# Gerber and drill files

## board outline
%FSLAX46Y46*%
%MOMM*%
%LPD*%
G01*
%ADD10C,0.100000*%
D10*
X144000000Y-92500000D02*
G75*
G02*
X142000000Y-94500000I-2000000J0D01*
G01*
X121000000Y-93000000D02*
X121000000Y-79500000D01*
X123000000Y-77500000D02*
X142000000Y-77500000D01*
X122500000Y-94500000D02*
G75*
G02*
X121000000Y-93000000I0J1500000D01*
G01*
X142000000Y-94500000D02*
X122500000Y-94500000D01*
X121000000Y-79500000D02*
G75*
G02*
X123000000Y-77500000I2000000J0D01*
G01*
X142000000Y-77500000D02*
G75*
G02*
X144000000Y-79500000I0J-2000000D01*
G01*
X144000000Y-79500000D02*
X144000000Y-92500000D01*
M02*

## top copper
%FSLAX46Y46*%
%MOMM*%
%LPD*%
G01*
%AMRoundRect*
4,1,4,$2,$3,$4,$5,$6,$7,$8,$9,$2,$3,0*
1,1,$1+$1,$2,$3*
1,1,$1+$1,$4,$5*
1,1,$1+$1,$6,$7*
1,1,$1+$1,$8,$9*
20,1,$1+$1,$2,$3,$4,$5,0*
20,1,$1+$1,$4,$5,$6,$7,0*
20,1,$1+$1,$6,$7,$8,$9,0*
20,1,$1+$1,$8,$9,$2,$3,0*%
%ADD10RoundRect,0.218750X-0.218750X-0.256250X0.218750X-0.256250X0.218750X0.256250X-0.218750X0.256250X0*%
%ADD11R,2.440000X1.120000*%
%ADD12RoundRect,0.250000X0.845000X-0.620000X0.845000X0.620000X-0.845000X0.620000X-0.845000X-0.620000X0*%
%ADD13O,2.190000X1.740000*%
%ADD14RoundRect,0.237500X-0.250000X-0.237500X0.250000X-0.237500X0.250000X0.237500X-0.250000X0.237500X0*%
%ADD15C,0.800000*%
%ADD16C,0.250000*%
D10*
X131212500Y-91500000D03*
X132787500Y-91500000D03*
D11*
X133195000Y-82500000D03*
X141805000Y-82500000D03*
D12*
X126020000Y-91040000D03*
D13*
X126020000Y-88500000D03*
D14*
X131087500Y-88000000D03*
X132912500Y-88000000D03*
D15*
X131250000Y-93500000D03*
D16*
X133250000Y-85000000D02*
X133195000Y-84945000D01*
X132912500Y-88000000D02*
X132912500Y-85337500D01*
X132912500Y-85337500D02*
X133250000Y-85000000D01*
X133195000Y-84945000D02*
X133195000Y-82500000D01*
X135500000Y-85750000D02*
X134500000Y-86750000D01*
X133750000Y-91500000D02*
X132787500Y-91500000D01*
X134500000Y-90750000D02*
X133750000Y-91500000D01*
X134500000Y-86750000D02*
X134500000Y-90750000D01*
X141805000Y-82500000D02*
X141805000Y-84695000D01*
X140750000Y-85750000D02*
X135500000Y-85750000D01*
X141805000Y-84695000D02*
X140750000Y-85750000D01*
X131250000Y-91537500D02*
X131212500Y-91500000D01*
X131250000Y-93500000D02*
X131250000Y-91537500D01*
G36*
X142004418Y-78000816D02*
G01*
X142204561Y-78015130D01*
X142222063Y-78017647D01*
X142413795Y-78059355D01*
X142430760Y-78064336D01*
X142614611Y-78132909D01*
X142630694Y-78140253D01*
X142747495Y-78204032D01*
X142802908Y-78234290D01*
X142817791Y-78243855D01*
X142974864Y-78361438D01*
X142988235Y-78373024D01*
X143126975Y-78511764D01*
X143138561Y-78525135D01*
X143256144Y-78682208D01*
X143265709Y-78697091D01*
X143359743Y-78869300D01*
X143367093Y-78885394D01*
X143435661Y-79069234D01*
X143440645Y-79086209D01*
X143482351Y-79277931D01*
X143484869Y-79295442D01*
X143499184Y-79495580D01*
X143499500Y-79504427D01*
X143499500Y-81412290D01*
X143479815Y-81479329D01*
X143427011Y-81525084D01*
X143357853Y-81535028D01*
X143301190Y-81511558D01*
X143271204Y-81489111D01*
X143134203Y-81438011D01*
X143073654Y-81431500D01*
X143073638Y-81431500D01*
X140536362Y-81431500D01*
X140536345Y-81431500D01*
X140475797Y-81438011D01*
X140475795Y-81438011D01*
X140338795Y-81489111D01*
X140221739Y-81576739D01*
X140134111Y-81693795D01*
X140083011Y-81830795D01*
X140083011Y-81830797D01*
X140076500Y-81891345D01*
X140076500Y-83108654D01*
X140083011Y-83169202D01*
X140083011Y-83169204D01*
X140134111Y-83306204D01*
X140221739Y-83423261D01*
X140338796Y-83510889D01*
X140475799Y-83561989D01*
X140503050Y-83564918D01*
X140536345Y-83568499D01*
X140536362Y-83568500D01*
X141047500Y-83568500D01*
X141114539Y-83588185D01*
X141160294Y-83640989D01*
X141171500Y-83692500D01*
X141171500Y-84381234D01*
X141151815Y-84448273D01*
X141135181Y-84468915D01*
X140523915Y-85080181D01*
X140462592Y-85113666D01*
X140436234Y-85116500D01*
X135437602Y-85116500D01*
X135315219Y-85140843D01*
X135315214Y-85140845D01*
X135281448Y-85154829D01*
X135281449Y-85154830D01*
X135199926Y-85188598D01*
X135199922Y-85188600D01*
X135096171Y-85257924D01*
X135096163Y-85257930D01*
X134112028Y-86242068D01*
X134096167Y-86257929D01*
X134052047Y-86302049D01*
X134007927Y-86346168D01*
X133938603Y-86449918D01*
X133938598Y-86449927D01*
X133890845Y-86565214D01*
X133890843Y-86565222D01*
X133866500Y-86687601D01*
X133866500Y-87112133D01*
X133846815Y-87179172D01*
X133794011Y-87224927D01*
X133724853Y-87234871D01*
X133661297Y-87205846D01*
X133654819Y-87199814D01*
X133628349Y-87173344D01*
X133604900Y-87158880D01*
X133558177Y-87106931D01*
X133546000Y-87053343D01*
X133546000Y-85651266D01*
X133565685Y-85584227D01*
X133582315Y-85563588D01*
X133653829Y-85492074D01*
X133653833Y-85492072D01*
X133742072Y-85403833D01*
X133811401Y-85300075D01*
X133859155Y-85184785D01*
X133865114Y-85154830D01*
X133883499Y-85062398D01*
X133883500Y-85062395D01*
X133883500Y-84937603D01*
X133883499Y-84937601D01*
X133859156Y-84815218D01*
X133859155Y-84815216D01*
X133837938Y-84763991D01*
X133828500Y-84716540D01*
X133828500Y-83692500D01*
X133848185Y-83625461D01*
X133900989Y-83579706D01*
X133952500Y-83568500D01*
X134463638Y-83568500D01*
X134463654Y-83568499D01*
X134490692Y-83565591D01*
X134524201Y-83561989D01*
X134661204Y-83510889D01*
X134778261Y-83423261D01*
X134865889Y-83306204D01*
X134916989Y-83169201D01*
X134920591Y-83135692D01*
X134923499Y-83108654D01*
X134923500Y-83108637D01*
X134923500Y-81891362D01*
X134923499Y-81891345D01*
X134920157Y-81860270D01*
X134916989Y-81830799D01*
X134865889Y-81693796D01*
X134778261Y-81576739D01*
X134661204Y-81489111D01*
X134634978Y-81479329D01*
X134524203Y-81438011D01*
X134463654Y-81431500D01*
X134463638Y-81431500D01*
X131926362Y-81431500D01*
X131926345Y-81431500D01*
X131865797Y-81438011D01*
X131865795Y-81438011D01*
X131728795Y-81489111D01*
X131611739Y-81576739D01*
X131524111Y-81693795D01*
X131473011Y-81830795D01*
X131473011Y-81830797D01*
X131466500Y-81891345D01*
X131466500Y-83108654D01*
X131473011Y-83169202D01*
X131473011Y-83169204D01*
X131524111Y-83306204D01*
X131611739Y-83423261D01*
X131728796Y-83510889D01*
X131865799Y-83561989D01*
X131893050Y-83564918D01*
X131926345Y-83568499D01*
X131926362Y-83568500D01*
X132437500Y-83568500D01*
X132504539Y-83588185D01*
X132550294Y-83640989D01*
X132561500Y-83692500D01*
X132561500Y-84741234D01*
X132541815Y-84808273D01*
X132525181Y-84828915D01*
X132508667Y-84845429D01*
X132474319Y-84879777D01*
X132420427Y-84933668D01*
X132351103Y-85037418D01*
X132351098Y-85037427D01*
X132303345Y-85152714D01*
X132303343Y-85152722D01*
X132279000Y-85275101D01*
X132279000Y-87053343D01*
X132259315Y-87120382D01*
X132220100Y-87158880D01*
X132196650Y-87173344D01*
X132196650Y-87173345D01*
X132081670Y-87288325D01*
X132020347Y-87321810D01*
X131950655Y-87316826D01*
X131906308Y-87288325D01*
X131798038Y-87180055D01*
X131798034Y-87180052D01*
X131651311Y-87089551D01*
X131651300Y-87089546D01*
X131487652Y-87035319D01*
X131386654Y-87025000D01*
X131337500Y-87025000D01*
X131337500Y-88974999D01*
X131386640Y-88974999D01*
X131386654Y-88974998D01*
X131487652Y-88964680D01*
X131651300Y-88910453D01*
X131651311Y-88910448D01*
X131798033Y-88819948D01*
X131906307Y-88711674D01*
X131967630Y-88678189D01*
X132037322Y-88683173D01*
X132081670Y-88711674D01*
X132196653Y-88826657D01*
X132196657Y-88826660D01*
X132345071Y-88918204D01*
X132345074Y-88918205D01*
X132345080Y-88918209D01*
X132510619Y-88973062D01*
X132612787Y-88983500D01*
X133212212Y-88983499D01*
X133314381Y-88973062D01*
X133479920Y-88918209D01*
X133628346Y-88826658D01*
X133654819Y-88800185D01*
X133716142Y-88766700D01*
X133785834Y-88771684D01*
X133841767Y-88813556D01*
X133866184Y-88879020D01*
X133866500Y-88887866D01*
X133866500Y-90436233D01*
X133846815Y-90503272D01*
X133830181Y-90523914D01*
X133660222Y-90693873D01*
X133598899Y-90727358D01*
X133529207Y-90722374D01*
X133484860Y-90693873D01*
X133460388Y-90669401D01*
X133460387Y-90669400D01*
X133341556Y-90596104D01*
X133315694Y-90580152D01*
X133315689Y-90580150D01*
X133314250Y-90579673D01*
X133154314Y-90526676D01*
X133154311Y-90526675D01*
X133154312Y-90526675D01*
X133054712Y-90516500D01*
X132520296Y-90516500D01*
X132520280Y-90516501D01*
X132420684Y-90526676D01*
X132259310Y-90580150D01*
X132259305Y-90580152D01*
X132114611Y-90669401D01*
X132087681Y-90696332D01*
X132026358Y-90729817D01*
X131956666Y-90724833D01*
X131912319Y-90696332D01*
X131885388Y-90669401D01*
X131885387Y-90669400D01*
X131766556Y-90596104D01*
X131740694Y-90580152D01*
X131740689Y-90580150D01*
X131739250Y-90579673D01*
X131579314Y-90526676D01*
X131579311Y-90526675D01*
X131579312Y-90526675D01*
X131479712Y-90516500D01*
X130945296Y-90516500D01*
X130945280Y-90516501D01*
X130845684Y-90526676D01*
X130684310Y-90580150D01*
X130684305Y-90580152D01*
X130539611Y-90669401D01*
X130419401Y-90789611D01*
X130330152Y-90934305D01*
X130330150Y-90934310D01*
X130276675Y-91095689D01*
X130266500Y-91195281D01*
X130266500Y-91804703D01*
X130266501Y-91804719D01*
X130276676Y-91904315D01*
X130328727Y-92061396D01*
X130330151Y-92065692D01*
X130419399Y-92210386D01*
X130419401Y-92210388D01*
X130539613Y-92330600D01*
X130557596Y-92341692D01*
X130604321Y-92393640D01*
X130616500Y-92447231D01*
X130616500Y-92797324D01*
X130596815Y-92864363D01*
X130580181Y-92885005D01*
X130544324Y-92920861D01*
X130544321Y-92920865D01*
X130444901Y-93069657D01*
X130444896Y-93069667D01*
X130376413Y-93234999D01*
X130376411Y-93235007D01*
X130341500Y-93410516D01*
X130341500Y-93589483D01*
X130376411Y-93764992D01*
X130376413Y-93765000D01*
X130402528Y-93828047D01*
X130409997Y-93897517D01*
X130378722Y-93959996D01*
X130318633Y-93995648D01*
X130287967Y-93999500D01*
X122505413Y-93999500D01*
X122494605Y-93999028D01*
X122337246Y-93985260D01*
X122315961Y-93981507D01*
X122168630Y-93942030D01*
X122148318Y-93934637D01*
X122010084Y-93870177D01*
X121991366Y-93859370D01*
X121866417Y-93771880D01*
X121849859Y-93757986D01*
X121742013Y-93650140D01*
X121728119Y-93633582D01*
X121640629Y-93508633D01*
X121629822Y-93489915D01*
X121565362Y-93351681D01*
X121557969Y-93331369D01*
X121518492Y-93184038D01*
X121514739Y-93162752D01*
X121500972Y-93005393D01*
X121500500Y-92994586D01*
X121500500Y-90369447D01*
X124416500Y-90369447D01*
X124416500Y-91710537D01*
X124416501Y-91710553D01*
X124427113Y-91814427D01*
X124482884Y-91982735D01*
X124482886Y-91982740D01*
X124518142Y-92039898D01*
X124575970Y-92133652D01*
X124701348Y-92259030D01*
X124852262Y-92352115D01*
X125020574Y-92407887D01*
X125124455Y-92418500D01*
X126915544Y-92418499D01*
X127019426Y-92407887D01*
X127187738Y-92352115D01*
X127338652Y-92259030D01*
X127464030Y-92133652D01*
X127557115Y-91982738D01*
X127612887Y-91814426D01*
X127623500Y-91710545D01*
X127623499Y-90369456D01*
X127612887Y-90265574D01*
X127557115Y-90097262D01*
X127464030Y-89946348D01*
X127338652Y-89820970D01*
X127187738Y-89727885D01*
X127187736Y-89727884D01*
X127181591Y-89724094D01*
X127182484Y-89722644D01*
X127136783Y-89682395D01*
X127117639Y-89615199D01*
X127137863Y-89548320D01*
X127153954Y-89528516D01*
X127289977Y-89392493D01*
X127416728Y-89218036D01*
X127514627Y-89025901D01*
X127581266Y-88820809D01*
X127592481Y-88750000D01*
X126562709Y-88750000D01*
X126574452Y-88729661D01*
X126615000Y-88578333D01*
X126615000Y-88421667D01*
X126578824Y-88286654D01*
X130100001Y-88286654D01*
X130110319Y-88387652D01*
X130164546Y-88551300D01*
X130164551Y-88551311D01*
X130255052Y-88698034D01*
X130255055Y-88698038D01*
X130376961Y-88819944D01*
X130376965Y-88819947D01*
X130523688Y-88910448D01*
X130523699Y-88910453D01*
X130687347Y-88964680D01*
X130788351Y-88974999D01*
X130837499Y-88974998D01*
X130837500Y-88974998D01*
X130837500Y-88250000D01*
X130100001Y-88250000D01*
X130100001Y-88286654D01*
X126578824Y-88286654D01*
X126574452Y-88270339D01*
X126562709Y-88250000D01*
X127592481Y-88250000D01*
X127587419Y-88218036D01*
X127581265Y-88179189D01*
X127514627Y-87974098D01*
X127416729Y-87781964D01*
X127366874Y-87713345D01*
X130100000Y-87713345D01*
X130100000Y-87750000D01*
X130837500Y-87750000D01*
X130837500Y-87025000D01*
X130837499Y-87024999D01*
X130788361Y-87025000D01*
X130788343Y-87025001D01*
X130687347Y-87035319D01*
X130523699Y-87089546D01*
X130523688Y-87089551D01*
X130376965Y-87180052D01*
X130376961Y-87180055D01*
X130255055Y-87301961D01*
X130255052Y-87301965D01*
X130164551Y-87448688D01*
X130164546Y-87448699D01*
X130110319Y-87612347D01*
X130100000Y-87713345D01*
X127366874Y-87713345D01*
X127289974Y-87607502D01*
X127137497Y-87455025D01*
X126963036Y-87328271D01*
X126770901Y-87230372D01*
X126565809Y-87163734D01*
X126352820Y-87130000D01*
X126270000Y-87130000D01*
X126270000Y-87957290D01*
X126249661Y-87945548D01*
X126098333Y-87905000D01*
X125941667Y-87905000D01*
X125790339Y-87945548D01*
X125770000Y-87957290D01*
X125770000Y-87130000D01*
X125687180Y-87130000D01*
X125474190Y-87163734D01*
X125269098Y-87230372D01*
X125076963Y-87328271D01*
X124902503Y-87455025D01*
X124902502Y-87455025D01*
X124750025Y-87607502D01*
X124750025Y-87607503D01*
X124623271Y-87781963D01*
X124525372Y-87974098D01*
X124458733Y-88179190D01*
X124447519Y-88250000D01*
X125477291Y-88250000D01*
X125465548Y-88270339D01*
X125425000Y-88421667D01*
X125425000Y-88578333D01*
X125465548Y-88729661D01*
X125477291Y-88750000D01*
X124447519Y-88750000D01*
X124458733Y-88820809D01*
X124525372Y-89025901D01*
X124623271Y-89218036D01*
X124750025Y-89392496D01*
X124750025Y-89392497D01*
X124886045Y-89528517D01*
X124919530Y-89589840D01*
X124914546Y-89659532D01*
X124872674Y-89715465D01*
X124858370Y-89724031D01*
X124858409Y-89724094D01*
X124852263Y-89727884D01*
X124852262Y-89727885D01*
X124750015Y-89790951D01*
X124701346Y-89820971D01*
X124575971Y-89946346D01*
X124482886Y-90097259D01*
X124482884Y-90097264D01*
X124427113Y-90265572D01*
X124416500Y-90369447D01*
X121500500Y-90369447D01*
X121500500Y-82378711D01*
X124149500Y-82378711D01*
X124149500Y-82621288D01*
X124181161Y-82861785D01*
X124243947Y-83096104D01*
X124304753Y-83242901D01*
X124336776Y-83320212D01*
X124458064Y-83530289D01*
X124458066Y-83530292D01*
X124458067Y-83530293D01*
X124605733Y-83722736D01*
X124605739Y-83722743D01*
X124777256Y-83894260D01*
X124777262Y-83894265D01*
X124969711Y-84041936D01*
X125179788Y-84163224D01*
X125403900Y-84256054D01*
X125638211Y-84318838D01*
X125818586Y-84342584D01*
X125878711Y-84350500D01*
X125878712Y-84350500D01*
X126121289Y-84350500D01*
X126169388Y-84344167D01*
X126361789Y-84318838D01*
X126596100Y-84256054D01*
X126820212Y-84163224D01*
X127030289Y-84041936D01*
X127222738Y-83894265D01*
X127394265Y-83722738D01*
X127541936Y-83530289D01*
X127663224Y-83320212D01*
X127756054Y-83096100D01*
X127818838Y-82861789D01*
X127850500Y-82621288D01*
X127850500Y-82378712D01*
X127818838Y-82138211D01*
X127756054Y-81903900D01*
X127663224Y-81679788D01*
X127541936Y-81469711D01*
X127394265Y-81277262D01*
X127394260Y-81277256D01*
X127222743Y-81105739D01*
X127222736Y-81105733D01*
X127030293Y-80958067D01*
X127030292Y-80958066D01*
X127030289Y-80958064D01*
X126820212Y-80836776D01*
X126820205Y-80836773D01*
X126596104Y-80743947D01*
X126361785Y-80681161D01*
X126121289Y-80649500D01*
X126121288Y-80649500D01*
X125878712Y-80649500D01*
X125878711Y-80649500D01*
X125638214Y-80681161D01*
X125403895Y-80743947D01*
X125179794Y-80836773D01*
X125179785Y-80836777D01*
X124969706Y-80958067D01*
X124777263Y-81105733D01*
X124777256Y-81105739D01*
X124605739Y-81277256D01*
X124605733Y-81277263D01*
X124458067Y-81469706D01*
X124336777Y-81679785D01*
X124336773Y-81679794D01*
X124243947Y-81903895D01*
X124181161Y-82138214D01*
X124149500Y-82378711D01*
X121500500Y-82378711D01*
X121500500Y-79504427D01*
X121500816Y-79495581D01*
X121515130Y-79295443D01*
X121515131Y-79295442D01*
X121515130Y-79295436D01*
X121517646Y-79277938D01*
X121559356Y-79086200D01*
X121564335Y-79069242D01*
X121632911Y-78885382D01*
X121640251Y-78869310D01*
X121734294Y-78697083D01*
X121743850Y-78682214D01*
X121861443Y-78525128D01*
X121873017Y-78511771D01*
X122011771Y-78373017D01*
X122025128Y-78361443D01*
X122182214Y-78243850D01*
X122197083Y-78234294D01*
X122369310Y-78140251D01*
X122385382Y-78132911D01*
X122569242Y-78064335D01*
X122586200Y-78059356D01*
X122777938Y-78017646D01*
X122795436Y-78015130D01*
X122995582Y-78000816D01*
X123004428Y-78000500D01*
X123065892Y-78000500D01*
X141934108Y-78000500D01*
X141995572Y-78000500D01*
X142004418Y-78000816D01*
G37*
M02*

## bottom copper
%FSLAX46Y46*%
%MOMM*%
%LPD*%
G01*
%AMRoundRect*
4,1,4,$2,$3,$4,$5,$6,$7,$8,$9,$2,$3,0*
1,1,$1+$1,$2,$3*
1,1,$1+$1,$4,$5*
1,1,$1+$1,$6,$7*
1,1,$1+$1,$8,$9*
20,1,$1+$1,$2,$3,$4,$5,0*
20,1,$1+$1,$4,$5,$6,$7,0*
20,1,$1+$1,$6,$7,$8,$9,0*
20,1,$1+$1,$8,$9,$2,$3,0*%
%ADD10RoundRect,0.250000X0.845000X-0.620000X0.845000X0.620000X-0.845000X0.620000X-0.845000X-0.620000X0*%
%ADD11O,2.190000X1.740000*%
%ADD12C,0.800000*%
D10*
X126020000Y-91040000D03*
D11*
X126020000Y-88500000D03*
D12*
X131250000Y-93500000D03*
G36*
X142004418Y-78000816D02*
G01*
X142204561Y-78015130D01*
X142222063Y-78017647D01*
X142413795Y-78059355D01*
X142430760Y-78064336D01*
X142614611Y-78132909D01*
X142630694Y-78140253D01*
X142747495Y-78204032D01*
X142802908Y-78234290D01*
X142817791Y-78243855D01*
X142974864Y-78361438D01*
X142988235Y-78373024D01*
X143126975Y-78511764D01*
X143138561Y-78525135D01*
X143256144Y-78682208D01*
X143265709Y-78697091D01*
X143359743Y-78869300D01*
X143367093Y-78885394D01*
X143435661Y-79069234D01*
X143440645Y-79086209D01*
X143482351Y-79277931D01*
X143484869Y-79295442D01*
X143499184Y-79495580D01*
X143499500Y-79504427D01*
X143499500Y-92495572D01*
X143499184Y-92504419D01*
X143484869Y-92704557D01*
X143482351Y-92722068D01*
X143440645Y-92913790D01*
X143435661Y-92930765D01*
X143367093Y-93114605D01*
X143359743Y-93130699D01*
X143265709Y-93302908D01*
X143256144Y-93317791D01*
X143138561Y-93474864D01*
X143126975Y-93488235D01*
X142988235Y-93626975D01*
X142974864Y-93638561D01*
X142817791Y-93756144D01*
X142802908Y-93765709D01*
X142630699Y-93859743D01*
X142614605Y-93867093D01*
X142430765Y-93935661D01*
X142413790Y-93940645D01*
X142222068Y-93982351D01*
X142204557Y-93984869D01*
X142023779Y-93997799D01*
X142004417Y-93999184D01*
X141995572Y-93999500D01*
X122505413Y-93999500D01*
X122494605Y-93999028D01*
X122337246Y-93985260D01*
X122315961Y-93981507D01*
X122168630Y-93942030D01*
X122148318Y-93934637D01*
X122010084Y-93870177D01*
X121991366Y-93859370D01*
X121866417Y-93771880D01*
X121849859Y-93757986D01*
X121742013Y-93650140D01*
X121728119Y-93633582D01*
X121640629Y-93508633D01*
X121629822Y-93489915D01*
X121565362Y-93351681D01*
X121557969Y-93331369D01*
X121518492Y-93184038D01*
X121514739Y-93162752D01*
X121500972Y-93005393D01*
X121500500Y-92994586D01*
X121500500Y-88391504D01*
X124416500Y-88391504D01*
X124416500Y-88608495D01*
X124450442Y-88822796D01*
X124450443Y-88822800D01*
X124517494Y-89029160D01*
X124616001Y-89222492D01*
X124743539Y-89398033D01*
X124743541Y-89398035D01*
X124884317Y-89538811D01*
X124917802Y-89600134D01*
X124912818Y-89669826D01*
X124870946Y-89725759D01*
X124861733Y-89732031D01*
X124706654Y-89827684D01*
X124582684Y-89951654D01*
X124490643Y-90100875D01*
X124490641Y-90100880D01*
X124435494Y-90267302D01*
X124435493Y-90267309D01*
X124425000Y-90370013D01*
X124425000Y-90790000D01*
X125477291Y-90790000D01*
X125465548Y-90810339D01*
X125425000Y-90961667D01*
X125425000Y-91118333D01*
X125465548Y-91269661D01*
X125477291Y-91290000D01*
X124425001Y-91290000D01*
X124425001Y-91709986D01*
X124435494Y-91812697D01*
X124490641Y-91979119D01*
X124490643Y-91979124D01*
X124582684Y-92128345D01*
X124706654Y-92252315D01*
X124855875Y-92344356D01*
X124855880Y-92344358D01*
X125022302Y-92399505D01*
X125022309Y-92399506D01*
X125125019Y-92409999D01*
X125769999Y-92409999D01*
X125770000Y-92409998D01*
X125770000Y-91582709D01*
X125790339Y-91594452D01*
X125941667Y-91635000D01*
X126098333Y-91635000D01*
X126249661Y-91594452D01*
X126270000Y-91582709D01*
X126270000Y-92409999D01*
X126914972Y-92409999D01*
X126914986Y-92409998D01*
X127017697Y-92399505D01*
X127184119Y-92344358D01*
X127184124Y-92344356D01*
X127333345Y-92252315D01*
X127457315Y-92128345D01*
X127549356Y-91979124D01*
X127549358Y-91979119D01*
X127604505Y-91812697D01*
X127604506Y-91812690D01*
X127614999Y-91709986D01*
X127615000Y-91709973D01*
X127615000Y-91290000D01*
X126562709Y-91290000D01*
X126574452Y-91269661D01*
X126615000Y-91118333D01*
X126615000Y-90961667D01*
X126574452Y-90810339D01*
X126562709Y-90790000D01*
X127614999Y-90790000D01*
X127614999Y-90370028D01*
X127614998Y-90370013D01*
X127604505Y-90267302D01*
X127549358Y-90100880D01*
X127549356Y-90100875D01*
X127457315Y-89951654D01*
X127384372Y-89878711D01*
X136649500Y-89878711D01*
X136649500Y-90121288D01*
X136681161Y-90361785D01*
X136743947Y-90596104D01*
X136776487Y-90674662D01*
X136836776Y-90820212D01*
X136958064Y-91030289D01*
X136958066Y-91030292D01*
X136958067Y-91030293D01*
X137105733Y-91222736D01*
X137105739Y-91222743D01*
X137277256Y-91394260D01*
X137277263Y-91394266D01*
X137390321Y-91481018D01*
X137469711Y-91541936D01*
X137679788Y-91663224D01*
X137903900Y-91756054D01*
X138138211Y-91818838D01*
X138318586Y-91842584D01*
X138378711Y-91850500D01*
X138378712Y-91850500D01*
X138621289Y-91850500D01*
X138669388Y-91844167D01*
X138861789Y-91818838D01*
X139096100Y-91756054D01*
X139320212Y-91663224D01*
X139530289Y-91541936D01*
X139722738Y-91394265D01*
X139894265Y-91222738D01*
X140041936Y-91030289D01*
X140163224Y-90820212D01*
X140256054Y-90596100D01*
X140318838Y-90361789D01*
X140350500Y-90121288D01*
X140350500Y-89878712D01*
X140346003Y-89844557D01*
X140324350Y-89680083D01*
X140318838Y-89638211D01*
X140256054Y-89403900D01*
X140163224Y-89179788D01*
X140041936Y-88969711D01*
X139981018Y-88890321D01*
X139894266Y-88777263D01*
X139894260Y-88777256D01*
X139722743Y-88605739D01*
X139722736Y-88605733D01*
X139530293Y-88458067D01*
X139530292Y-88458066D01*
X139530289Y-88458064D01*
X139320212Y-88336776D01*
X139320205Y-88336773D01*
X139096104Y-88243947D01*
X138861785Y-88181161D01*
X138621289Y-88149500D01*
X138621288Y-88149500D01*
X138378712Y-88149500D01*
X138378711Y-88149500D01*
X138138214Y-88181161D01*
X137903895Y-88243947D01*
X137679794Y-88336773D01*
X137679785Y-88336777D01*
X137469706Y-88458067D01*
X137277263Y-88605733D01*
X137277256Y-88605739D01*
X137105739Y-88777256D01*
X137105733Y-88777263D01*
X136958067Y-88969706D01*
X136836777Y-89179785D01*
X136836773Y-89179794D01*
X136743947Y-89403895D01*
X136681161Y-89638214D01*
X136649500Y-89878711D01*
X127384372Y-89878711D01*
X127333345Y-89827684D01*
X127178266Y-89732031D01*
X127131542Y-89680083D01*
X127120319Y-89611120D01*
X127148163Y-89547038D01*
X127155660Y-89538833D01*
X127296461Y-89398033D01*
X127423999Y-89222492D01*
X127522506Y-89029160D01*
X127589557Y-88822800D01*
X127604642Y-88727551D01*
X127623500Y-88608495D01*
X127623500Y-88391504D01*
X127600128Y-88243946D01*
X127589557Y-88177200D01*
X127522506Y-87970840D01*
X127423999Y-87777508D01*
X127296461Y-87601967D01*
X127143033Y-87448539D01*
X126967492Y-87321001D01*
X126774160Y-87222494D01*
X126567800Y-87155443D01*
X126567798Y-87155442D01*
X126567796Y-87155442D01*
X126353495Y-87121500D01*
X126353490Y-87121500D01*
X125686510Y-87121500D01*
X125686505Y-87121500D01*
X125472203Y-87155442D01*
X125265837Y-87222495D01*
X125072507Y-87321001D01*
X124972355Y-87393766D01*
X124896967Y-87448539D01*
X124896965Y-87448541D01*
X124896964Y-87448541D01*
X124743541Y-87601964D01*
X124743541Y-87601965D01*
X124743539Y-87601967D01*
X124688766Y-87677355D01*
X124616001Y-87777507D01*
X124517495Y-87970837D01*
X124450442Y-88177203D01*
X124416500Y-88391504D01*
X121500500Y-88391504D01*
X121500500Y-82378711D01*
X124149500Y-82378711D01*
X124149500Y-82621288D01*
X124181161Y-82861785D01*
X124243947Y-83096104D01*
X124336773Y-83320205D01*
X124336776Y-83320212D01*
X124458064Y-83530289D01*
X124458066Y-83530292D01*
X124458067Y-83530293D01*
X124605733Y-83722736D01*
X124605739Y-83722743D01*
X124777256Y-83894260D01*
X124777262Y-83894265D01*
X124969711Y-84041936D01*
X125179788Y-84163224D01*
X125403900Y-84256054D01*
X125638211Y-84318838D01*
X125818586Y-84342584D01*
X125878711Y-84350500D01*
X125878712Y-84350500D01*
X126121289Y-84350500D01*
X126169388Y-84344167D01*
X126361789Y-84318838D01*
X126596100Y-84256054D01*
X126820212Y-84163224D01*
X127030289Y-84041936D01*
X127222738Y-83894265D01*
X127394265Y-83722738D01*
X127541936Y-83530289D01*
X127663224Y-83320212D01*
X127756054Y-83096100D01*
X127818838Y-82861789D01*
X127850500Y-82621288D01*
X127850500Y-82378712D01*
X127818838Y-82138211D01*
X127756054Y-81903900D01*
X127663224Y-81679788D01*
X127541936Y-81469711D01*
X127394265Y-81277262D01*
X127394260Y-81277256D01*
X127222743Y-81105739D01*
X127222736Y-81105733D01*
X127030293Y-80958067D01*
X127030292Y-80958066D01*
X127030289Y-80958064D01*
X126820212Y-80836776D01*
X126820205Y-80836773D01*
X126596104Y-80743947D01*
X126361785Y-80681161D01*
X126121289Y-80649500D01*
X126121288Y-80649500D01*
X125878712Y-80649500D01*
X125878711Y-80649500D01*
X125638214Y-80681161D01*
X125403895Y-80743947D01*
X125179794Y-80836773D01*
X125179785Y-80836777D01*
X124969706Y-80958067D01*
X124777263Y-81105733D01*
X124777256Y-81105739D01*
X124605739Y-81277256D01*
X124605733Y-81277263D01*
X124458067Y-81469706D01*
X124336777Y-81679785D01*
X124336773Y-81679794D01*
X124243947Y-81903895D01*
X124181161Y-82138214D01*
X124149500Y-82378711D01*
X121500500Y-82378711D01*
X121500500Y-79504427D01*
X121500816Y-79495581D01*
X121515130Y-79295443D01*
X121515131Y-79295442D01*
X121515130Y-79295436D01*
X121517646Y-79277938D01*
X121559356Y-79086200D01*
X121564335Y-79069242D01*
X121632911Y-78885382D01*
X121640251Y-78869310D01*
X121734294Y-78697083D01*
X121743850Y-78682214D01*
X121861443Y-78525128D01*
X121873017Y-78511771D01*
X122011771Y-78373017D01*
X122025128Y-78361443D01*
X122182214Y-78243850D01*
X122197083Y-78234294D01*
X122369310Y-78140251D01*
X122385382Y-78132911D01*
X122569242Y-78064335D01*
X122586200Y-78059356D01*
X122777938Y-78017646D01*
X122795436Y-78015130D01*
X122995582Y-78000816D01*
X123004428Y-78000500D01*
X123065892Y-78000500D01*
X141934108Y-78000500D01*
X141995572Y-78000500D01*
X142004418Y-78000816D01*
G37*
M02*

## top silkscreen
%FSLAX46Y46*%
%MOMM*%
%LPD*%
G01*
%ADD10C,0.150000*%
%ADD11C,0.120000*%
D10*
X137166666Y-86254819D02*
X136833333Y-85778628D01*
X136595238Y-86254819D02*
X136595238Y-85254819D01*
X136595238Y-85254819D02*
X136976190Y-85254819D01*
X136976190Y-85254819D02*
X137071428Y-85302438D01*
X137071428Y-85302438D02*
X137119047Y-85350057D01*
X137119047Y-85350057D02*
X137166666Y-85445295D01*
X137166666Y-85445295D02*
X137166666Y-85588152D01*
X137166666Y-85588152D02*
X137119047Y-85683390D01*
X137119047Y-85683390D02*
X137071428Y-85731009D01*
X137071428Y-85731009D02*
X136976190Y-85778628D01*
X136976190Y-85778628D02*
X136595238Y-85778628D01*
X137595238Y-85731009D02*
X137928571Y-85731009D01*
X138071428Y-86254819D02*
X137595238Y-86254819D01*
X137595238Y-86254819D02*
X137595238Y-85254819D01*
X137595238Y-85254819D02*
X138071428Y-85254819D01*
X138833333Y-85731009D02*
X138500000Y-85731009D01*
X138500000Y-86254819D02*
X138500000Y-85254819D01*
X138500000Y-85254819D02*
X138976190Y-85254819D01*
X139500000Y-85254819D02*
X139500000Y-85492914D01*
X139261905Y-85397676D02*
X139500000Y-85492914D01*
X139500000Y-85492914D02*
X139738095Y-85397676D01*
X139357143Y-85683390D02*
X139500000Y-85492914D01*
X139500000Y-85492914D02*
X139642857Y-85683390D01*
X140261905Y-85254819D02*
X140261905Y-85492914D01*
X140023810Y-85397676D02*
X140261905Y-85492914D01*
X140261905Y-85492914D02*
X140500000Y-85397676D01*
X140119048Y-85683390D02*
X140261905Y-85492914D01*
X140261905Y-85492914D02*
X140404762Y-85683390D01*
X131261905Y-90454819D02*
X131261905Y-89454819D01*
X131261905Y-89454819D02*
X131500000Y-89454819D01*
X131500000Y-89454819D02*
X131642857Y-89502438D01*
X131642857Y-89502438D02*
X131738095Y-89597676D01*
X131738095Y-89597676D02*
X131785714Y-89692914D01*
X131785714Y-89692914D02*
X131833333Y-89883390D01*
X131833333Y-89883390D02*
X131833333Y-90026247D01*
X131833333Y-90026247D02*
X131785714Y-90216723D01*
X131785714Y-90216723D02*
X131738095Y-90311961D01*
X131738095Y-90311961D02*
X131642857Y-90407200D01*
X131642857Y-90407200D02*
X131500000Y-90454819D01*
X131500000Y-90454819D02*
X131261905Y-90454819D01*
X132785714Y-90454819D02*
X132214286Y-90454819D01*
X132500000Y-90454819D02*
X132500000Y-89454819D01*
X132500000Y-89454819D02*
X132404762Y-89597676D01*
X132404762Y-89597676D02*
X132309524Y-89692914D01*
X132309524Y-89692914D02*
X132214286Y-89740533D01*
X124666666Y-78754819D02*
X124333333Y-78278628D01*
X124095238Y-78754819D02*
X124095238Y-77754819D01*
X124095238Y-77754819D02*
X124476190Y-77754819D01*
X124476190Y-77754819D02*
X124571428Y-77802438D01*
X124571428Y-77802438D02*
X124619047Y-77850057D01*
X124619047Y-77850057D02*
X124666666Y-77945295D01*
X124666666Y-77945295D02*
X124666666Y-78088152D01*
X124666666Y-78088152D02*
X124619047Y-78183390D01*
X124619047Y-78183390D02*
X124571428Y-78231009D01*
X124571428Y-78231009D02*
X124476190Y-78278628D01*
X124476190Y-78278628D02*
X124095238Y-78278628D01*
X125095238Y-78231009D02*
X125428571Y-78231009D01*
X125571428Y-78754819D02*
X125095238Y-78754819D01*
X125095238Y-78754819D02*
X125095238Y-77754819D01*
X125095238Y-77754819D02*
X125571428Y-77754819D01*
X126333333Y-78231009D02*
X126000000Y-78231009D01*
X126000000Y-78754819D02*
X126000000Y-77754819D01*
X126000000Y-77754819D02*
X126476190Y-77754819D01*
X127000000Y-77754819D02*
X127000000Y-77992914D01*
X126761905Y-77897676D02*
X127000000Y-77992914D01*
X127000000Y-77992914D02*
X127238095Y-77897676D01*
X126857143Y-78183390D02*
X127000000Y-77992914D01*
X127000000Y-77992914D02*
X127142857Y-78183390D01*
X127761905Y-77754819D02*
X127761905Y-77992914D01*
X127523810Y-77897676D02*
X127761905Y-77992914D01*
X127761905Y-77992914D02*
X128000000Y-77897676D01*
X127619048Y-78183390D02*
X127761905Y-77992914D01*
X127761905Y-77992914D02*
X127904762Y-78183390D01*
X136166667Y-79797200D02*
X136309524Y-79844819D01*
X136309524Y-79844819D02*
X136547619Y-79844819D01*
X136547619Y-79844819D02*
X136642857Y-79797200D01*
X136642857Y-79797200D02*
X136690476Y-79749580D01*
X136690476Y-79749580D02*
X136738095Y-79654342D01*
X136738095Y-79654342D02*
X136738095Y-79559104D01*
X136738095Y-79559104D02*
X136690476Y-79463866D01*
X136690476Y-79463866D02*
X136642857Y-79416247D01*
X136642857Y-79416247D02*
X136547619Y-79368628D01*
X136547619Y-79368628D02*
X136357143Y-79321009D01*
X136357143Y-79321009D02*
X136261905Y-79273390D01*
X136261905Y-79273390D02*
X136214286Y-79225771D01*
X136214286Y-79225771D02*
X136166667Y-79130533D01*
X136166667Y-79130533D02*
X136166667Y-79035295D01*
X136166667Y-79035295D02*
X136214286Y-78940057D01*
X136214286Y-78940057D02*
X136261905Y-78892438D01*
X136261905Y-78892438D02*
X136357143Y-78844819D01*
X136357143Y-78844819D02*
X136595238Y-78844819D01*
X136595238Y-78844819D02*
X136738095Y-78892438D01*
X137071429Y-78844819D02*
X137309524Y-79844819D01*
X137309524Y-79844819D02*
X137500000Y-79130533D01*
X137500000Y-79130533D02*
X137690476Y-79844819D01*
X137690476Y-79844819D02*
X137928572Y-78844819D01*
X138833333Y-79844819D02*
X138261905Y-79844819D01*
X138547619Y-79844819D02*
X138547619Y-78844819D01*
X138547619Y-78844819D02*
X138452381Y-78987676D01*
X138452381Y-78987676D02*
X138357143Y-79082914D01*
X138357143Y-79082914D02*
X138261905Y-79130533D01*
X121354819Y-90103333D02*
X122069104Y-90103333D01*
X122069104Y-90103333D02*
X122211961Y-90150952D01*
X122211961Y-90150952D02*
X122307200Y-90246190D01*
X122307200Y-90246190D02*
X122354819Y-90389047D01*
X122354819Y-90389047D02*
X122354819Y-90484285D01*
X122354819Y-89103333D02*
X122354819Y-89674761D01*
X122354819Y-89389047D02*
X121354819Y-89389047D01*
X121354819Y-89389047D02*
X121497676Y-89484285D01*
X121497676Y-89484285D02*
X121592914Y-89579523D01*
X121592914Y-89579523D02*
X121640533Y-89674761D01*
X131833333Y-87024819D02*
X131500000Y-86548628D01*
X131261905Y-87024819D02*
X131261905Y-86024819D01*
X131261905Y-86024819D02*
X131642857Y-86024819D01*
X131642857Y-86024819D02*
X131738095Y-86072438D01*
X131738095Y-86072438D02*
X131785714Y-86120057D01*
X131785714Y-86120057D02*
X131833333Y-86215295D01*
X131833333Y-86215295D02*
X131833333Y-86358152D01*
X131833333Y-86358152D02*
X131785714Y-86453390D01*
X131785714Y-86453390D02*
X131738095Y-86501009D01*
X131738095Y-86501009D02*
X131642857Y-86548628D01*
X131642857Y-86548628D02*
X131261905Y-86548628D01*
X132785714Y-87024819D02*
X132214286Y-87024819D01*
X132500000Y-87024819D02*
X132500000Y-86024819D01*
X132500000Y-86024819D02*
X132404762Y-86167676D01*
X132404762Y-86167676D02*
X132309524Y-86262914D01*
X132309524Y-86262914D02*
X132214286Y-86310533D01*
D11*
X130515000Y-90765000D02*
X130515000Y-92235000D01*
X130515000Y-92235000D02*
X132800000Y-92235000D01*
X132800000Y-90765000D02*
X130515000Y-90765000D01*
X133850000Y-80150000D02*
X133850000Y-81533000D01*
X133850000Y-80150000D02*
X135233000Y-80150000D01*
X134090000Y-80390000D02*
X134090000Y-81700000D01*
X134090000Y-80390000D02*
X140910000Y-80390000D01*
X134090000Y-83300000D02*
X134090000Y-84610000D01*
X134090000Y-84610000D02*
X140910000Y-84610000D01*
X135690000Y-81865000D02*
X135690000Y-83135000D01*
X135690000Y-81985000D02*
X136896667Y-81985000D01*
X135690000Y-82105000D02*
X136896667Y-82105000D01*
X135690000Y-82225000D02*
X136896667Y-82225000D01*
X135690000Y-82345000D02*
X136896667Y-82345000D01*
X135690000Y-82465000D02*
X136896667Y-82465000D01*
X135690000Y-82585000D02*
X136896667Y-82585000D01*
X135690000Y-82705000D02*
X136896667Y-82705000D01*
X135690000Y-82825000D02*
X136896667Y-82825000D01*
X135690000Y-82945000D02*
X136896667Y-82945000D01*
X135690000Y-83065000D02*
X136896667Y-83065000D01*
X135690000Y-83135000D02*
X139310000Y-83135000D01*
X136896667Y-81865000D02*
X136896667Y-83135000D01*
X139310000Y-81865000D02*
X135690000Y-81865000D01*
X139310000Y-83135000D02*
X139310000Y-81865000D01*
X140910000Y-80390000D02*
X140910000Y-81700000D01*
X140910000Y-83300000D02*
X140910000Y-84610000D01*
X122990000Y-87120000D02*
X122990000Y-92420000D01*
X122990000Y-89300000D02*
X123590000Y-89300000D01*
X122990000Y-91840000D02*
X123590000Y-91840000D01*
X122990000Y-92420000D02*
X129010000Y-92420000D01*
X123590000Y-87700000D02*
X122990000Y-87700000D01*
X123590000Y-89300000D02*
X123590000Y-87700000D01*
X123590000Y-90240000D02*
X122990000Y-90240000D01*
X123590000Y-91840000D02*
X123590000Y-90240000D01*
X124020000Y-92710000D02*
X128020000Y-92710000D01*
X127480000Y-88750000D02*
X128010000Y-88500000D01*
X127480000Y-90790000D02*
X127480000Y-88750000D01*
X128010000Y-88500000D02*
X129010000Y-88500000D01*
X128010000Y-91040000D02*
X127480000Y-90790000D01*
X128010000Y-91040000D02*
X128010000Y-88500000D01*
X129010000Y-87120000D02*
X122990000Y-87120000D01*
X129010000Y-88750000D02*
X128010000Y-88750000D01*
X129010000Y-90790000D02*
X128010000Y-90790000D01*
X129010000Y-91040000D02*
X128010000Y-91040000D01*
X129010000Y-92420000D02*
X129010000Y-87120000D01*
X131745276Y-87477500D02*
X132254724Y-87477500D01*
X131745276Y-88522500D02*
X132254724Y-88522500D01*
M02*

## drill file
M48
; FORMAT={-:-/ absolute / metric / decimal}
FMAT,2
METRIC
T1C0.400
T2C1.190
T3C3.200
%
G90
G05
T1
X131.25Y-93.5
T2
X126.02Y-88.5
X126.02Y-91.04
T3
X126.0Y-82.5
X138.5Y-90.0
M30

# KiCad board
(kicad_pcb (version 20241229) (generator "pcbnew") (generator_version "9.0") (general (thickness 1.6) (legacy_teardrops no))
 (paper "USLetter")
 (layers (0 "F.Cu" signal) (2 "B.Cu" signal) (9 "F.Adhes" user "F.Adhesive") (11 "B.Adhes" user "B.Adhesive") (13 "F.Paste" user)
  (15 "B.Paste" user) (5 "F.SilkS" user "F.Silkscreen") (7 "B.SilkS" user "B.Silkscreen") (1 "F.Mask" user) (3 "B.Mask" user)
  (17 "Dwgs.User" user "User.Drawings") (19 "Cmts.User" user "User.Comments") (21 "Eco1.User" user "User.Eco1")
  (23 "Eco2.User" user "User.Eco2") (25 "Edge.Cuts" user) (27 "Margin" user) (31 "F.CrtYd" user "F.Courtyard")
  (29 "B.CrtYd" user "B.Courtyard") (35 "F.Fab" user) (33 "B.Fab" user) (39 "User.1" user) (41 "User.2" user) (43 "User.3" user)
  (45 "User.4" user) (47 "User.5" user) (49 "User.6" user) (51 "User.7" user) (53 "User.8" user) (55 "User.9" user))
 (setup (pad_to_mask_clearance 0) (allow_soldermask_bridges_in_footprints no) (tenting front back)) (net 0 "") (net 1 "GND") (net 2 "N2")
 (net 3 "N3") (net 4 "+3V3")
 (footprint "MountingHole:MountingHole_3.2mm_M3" (layer "F.Cu") (at 138.5 90)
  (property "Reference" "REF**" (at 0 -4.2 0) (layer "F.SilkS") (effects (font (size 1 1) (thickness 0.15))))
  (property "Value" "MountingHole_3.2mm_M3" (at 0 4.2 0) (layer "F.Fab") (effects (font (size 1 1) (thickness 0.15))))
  (pad "" np_thru_hole circle (at 0 0) (size 3.2 3.2) (drill 3.2) (layers "*.Cu" "*.Mask")))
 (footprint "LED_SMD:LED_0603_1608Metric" (layer "F.Cu") (at 132 91.5)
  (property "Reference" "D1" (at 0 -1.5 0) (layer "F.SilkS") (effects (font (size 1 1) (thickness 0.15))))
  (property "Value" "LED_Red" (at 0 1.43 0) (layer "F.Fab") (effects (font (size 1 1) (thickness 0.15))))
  (fp_line (start -1.485 -0.735) (end -1.485 0.735) (stroke (width 0.12) (type solid)) (layer "F.SilkS"))
  (fp_line (start -1.485 0.735) (end 0.8 0.735) (stroke (width 0.12) (type solid)) (layer "F.SilkS"))
  (fp_line (start 0.8 -0.735) (end -1.485 -0.735) (stroke (width 0.12) (type solid)) (layer "F.SilkS"))
  (pad "1" smd roundrect (at -0.7875 0) (size 0.875 0.95) (layers "F.Cu" "F.Mask" "F.Paste") (roundrect_rratio 0.25) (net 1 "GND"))
  (pad "2" smd roundrect (at 0.7875 0) (size 0.875 0.95) (layers "F.Cu" "F.Mask" "F.Paste") (roundrect_rratio 0.25) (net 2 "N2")))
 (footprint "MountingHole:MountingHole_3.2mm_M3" (layer "F.Cu") (at 126 82.5)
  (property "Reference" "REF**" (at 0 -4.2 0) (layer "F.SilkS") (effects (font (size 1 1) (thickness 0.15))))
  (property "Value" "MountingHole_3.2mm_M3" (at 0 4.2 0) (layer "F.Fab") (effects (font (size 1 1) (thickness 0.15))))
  (pad "" np_thru_hole circle (at 0 0) (size 3.2 3.2) (drill 3.2) (layers "*.Cu" "*.Mask")))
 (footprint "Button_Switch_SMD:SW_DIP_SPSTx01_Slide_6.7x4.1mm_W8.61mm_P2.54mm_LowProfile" (layer "F.Cu") (at 137.5 82.5)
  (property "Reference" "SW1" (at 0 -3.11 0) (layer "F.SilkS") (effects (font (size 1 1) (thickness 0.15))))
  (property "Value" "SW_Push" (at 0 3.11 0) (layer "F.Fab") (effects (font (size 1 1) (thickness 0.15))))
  (fp_line (start -3.65 -2.35) (end -3.65 -0.967) (stroke (width 0.12) (type solid)) (layer "F.SilkS"))
  (fp_line (start -3.65 -2.35) (end -2.267 -2.35) (stroke (width 0.12) (type solid)) (layer "F.SilkS"))
  (fp_line (start -3.41 -2.11) (end -3.41 -0.8) (stroke (width 0.12) (type solid)) (layer "F.SilkS"))
  (fp_line (start -3.41 -2.11) (end 3.41 -2.11) (stroke (width 0.12) (type solid)) (layer "F.SilkS"))
  (fp_line (start -3.41 0.8) (end -3.41 2.11) (stroke (width 0.12) (type solid)) (layer "F.SilkS"))
  (fp_line (start -3.41 2.11) (end 3.41 2.11) (stroke (width 0.12) (type solid)) (layer "F.SilkS"))
  (fp_line (start -1.81 -0.635) (end -1.81 0.635) (stroke (width 0.12) (type solid)) (layer "F.SilkS"))
  (fp_line (start -1.81 -0.515) (end -0.603333 -0.515) (stroke (width 0.12) (type solid)) (layer "F.SilkS"))
  (fp_line (start -1.81 -0.395) (end -0.603333 -0.395) (stroke (width 0.12) (type solid)) (layer "F.SilkS"))
  (fp_line (start -1.81 -0.275) (end -0.603333 -0.275) (stroke (width 0.12) (type solid)) (layer "F.SilkS"))
  (fp_line (start -1.81 -0.155) (end -0.603333 -0.155) (stroke (width 0.12) (type solid)) (layer "F.SilkS"))
  (fp_line (start -1.81 -0.035) (end -0.603333 -0.035) (stroke (width 0.12) (type solid)) (layer "F.SilkS"))
  (fp_line (start -1.81 0.085) (end -0.603333 0.085) (stroke (width 0.12) (type solid)) (layer "F.SilkS"))
  (fp_line (start -1.81 0.205) (end -0.603333 0.205) (stroke (width 0.12) (type solid)) (layer "F.SilkS"))
  (fp_line (start -1.81 0.325) (end -0.603333 0.325) (stroke (width 0.12) (type solid)) (layer "F.SilkS"))
  (fp_line (start -1.81 0.445) (end -0.603333 0.445) (stroke (width 0.12) (type solid)) (layer "F.SilkS"))
  (fp_line (start -1.81 0.565) (end -0.603333 0.565) (stroke (width 0.12) (type solid)) (layer "F.SilkS"))
  (fp_line (start -1.81 0.635) (end 1.81 0.635) (stroke (width 0.12) (type solid)) (layer "F.SilkS"))
  (fp_line (start -0.603333 -0.635) (end -0.603333 0.635) (stroke (width 0.12) (type solid)) (layer "F.SilkS"))
  (fp_line (start 1.81 -0.635) (end -1.81 -0.635) (stroke (width 0.12) (type solid)) (layer "F.SilkS"))
  (fp_line (start 1.81 0.635) (end 1.81 -0.635) (stroke (width 0.12) (type solid)) (layer "F.SilkS"))
  (fp_line (start 3.41 -2.11) (end 3.41 -0.8) (stroke (width 0.12) (type solid)) (layer "F.SilkS"))
  (fp_line (start 3.41 0.8) (end 3.41 2.11) (stroke (width 0.12) (type solid)) (layer "F.SilkS"))
  (pad "1" smd rect (at -4.305 0) (size 2.44 1.12) (layers "F.Cu" "F.Mask" "F.Paste") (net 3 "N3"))
  (pad "2" smd rect (at 4.305 0) (size 2.44 1.12) (layers "F.Cu" "F.Mask" "F.Paste") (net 2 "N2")))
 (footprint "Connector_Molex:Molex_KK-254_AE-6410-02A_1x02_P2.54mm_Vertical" (layer "F.Cu") (at 126.02 91.04 90)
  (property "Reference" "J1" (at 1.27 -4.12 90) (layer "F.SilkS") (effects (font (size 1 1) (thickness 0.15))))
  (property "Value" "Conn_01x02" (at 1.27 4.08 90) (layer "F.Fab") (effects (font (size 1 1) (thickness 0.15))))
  (fp_line (start 3.92 -3.03) (end -1.38 -3.03) (stroke (width 0.12) (type solid)) (layer "F.SilkS"))
  (fp_line (start 1.74 -3.03) (end 1.74 -2.43) (stroke (width 0.12) (type solid)) (layer "F.SilkS"))
  (fp_line (start -0.8 -3.03) (end -0.8 -2.43) (stroke (width 0.12) (type solid)) (layer "F.SilkS"))
  (fp_line (start -1.38 -3.03) (end -1.38 2.99) (stroke (width 0.12) (type solid)) (layer "F.SilkS"))
  (fp_line (start 3.34 -2.43) (end 3.34 -3.03) (stroke (width 0.12) (type solid)) (layer "F.SilkS"))
  (fp_line (start 1.74 -2.43) (end 3.34 -2.43) (stroke (width 0.12) (type solid)) (layer "F.SilkS"))
  (fp_line (start 0.8 -2.43) (end 0.8 -3.03) (stroke (width 0.12) (type solid)) (layer "F.SilkS"))
  (fp_line (start -0.8 -2.43) (end 0.8 -2.43) (stroke (width 0.12) (type solid)) (layer "F.SilkS"))
  (fp_line (start -1.67 -2) (end -1.67 2) (stroke (width 0.12) (type solid)) (layer "F.SilkS"))
  (fp_line (start 2.29 1.46) (end 2.54 1.99) (stroke (width 0.12) (type solid)) (layer "F.SilkS"))
  (fp_line (start 0.25 1.46) (end 2.29 1.46) (stroke (width 0.12) (type solid)) (layer "F.SilkS"))
  (fp_line (start 2.54 1.99) (end 2.54 2.99) (stroke (width 0.12) (type solid)) (layer "F.SilkS"))
  (fp_line (start 0 1.99) (end 0.25 1.46) (stroke (width 0.12) (type solid)) (layer "F.SilkS"))
  (fp_line (start 0 1.99) (end 2.54 1.99) (stroke (width 0.12) (type solid)) (layer "F.SilkS"))
  (fp_line (start 3.92 2.99) (end 3.92 -3.03) (stroke (width 0.12) (type solid)) (layer "F.SilkS"))
  (fp_line (start 2.29 2.99) (end 2.29 1.99) (stroke (width 0.12) (type solid)) (layer "F.SilkS"))
  (fp_line (start 0.25 2.99) (end 0.25 1.99) (stroke (width 0.12) (type solid)) (layer "F.SilkS"))
  (fp_line (start 0 2.99) (end 0 1.99) (stroke (width 0.12) (type solid)) (layer "F.SilkS"))
  (fp_line (start -1.38 2.99) (end 3.92 2.99) (stroke (width 0.12) (type solid)) (layer "F.SilkS"))
  (pad "1" thru_hole roundrect (at 0 0 90) (size 1.74 2.19) (drill 1.19) (layers "*.Cu" "*.Mask") (remove_unused_layers no)
   (roundrect_rratio 0.143678) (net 1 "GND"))
  (pad "2" thru_hole oval (at 2.54 0 90) (size 1.74 2.19) (drill 1.19) (layers "*.Cu" "*.Mask") (remove_unused_layers no) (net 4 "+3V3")))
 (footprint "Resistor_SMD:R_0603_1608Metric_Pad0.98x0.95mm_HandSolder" (layer "F.Cu") (at 132 88)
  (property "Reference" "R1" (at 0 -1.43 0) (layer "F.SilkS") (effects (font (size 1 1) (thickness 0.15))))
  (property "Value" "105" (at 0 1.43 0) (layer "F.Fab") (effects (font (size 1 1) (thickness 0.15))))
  (fp_line (start -0.254724 -0.5225) (end 0.254724 -0.5225) (stroke (width 0.12) (type solid)) (layer "F.SilkS"))
  (fp_line (start -0.254724 0.5225) (end 0.254724 0.5225) (stroke (width 0.12) (type solid)) (layer "F.SilkS"))
  (pad "1" smd roundrect (at -0.9125 0) (size 0.975 0.95) (layers "F.Cu" "F.Mask" "F.Paste") (roundrect_rratio 0.25) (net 4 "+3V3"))
  (pad "2" smd roundrect (at 0.9125 0) (size 0.975 0.95) (layers "F.Cu" "F.Mask" "F.Paste") (roundrect_rratio 0.25) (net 3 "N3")))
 (gr_arc (start 144 92.5) (mid 143.414214 93.914214) (end 142 94.5) (stroke (width 0.1) (type default)) (layer "Edge.Cuts"))
 (gr_line (start 121 93) (end 121 79.5) (stroke (width 0.1) (type default)) (layer "Edge.Cuts"))
 (gr_line (start 123 77.5) (end 142 77.5) (stroke (width 0.1) (type default)) (layer "Edge.Cuts"))
 (gr_arc (start 122.5 94.5) (mid 121.43934 94.06066) (end 121 93) (stroke (width 0.1) (type default)) (layer "Edge.Cuts"))
 (gr_line (start 142 94.5) (end 122.5 94.5) (stroke (width 0.1) (type default)) (layer "Edge.Cuts"))
 (gr_arc (start 121 79.5) (mid 121.585786 78.085786) (end 123 77.5) (stroke (width 0.1) (type default)) (layer "Edge.Cuts"))
 (gr_arc (start 142 77.5) (mid 143.414214 78.085786) (end 144 79.5) (stroke (width 0.1) (type default)) (layer "Edge.Cuts"))
 (gr_line (start 144 79.5) (end 144 92.5) (stroke (width 0.1) (type default)) (layer "Edge.Cuts"))
 (segment (start 133.25 85) (end 133.195 84.945) (width 0.25) (layer "F.Cu") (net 3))
 (segment (start 132.9125 88) (end 132.9125 85.3375) (width 0.25) (layer "F.Cu") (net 3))
 (segment (start 132.9125 85.3375) (end 133.25 85) (width 0.25) (layer "F.Cu") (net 3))
 (segment (start 133.195 84.945) (end 133.195 82.5) (width 0.25) (layer "F.Cu") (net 3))
 (segment (start 135.5 85.75) (end 134.5 86.75) (width 0.25) (layer "F.Cu") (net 2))
 (segment (start 133.75 91.5) (end 132.7875 91.5) (width 0.25) (layer "F.Cu") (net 2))
 (segment (start 134.5 90.75) (end 133.75 91.5) (width 0.25) (layer "F.Cu") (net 2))
 (segment (start 134.5 86.75) (end 134.5 90.75) (width 0.25) (layer "F.Cu") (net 2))
 (segment (start 141.805 82.5) (end 141.805 84.695) (width 0.25) (layer "F.Cu") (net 2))
 (segment (start 140.75 85.75) (end 135.5 85.75) (width 0.25) (layer "F.Cu") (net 2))
 (segment (start 141.805 84.695) (end 140.75 85.75) (width 0.25) (layer "F.Cu") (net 2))
 (segment (start 131.25 91.5375) (end 131.2125 91.5) (width 0.25) (layer "F.Cu") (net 1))
 (segment (start 131.25 93.5) (end 131.25 91.5375) (width 0.25) (layer "F.Cu") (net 1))
 (via (at 131.25 93.5) (size 0.8) (drill 0.4) (layers "F.Cu" "B.Cu") (free yes) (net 1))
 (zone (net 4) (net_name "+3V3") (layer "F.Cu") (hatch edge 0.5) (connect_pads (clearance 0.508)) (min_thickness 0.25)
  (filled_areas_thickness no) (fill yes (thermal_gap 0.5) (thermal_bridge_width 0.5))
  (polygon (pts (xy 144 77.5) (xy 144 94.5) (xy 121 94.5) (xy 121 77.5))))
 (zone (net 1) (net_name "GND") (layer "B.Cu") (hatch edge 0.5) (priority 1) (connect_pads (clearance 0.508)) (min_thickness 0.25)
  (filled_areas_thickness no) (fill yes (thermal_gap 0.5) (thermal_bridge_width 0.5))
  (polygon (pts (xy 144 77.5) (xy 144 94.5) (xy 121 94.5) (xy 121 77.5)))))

